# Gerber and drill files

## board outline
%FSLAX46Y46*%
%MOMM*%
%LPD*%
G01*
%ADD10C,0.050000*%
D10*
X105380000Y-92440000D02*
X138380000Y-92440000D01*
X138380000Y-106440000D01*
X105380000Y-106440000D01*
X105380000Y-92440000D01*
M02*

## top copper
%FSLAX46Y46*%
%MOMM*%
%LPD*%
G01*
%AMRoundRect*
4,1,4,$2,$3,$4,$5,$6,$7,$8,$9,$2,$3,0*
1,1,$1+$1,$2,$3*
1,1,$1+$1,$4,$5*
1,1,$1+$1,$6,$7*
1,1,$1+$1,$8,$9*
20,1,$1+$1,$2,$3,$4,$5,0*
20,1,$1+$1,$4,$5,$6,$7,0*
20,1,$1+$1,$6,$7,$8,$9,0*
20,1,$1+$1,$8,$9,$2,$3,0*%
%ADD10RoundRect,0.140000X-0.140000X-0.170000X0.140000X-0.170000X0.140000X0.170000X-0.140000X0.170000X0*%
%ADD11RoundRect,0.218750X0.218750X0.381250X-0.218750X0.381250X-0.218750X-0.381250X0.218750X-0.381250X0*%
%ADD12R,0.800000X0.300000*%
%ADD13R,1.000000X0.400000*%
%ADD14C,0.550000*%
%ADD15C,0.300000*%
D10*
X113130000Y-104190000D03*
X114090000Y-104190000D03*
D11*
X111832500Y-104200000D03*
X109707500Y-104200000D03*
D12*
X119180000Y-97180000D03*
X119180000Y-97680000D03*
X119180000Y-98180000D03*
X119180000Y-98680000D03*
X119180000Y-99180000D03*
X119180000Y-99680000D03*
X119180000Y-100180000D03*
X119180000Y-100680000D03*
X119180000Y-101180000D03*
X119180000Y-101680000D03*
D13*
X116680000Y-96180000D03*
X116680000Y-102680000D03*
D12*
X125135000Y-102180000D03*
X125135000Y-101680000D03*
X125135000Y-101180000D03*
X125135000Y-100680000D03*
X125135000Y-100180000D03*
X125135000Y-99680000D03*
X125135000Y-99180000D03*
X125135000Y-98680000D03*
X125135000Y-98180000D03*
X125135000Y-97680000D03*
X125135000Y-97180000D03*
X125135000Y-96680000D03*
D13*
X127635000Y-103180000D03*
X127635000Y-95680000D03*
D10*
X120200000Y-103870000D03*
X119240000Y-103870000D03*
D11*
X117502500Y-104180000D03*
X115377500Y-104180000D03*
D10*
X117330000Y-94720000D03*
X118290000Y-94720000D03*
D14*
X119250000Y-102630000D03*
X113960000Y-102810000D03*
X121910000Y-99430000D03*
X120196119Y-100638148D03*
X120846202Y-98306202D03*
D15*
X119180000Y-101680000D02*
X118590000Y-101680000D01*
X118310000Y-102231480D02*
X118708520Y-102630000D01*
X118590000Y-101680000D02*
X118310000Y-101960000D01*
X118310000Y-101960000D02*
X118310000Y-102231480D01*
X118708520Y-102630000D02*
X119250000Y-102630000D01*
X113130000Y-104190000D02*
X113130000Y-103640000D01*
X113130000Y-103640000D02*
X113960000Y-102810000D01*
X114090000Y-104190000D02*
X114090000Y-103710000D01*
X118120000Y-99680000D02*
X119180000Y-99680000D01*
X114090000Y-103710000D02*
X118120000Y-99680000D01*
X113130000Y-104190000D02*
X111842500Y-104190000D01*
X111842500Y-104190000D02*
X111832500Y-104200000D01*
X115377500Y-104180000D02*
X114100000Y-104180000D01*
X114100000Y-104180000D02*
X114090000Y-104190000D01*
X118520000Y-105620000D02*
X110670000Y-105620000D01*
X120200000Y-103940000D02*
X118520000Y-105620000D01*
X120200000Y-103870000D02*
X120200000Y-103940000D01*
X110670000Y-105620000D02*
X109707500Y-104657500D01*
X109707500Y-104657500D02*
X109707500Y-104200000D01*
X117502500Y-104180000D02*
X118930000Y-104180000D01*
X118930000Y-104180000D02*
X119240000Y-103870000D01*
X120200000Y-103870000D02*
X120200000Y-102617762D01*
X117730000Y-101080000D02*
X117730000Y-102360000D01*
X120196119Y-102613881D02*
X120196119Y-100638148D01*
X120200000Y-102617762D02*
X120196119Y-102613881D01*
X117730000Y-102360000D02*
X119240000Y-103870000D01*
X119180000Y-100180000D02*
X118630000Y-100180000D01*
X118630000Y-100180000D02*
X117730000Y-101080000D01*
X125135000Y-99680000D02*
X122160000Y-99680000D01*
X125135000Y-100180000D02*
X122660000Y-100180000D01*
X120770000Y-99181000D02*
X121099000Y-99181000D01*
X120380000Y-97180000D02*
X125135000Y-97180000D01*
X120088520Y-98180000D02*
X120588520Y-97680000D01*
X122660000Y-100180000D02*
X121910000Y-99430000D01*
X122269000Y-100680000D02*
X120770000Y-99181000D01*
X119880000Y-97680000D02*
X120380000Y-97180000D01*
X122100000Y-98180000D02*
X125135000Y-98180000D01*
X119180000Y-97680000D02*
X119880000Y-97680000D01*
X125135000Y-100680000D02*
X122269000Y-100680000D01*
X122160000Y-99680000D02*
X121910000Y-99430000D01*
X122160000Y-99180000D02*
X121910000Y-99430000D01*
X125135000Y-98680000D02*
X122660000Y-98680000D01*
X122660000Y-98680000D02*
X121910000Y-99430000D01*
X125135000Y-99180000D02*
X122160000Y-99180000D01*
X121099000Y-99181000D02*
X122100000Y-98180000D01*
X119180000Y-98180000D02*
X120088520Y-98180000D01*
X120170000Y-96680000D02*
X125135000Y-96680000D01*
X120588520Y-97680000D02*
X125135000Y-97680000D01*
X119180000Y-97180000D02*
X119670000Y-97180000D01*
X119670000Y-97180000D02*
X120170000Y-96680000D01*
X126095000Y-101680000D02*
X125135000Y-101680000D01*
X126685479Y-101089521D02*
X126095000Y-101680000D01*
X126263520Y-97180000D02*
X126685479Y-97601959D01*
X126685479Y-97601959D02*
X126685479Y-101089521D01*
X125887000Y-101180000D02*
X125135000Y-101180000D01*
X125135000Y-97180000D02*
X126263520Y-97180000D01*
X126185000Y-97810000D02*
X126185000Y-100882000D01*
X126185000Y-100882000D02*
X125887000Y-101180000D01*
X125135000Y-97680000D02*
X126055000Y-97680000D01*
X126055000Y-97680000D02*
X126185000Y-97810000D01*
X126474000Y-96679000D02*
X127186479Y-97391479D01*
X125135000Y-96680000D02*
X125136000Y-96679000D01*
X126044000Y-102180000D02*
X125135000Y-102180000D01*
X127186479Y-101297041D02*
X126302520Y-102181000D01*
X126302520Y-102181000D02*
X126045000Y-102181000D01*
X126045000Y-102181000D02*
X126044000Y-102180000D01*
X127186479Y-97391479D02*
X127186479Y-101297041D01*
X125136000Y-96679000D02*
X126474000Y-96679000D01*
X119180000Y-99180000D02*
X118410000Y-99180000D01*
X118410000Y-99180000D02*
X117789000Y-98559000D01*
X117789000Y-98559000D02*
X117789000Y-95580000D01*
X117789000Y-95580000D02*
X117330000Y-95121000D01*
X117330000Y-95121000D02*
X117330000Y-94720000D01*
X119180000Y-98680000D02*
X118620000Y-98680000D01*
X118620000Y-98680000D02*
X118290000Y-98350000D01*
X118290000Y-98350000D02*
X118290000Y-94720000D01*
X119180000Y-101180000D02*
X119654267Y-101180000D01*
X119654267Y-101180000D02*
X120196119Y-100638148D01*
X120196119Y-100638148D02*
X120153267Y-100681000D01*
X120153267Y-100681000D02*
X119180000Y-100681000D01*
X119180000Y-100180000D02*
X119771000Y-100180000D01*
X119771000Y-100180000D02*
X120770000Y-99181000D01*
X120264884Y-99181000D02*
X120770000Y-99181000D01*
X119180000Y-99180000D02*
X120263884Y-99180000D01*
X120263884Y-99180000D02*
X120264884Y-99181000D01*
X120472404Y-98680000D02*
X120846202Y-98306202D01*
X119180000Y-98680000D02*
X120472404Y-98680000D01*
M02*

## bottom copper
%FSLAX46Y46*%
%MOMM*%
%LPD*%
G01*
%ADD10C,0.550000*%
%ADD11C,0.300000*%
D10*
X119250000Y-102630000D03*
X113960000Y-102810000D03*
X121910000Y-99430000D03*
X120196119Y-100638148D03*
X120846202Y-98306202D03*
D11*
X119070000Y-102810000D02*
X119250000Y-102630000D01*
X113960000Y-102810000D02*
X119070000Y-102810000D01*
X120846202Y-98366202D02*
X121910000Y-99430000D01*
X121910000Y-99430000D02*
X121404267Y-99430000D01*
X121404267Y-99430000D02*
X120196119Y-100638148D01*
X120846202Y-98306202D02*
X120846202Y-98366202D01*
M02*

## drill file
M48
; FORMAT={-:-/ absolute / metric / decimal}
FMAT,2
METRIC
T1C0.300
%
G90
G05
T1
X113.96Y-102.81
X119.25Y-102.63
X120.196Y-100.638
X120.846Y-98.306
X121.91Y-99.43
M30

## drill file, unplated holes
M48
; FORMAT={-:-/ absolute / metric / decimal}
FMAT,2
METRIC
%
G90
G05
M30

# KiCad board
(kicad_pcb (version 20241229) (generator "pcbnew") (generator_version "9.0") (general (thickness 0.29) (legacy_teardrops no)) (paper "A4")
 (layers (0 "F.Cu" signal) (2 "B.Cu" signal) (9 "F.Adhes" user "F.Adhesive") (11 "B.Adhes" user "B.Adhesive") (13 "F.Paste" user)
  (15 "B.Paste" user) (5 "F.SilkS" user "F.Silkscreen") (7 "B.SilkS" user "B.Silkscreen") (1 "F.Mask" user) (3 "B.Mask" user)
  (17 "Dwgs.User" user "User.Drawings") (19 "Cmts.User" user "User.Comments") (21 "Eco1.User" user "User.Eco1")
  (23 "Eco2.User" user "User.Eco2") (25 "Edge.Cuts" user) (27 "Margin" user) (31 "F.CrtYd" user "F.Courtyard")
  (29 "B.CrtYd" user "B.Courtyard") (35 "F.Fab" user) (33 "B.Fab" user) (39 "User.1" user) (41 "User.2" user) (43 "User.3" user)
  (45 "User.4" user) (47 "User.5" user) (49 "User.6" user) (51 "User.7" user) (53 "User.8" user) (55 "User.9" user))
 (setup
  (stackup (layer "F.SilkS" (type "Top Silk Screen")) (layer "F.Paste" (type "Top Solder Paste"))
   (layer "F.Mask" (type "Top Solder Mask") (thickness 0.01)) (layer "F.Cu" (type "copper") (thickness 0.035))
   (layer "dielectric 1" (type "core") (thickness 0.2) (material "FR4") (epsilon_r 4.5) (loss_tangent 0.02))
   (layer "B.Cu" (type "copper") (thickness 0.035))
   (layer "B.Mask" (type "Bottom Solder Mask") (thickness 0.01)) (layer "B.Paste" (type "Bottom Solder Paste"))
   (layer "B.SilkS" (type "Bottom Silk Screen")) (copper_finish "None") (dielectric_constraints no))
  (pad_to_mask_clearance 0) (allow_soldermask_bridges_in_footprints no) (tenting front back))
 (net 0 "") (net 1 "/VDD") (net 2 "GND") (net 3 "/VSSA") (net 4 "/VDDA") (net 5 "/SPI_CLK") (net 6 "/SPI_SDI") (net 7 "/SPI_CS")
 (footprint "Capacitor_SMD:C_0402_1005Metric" (layer "F.Cu") (at 119.72 103.87)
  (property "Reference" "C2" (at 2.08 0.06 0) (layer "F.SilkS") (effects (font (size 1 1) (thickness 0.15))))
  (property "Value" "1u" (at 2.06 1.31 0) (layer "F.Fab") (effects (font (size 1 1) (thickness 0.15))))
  (pad "1" smd roundrect (at -0.48 0) (size 0.56 0.62) (layers "F.Cu" "F.Mask" "F.Paste") (roundrect_rratio 0.25) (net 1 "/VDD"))
  (pad "2" smd roundrect (at 0.48 0) (size 0.56 0.62) (layers "F.Cu" "F.Mask" "F.Paste") (roundrect_rratio 0.25) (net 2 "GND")))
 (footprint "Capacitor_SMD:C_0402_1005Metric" (layer "F.Cu") (at 113.61 104.19)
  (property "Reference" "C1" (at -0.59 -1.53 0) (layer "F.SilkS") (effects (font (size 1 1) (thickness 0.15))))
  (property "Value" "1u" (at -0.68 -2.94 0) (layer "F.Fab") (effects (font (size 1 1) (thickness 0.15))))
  (pad "1" smd roundrect (at -0.48 0) (size 0.56 0.62) (layers "F.Cu" "F.Mask" "F.Paste") (roundrect_rratio 0.25) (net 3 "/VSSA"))
  (pad "2" smd roundrect (at 0.48 0) (size 0.56 0.62) (layers "F.Cu" "F.Mask" "F.Paste") (roundrect_rratio 0.25) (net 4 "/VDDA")))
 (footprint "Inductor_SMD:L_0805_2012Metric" (layer "F.Cu") (at 116.44 104.18 180)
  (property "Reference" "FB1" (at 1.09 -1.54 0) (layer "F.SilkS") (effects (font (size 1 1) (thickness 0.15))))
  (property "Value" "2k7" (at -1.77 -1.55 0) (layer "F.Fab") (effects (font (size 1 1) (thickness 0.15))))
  (pad "1" smd roundrect (at -1.0625 0 180) (size 0.875 1.2) (layers "F.Cu" "F.Mask" "F.Paste") (roundrect_rratio 0.25) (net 1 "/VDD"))
  (pad "2" smd roundrect (at 1.0625 0 180) (size 0.875 1.2) (layers "F.Cu" "F.Mask" "F.Paste") (roundrect_rratio 0.25) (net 4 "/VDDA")))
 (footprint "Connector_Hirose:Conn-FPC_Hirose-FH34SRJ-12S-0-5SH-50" (layer "F.Cu") (at 126.16 99.43 90)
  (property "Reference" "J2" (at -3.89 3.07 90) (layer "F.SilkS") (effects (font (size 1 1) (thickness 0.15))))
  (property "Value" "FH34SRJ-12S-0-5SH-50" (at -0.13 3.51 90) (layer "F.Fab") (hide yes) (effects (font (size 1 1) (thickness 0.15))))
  (pad "1" smd rect (at -2.75 -1.025 90) (size 0.3 0.8) (layers "F.Cu" "F.Mask" "F.Paste") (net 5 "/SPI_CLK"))
  (pad "2" smd rect (at -2.25 -1.025 90) (size 0.3 0.8) (layers "F.Cu" "F.Mask" "F.Paste") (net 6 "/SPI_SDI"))
  (pad "3" smd rect (at -1.75 -1.025 90) (size 0.3 0.8) (layers "F.Cu" "F.Mask" "F.Paste") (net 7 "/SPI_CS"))
  (pad "4" smd rect (at -1.25 -1.025 90) (size 0.3 0.8) (layers "F.Cu" "F.Mask" "F.Paste") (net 1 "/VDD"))
  (pad "5" smd rect (at -0.75 -1.025 90) (size 0.3 0.8) (layers "F.Cu" "F.Mask" "F.Paste") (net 2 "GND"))
  (pad "6" smd rect (at -0.25 -1.025 90) (size 0.3 0.8) (layers "F.Cu" "F.Mask" "F.Paste") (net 2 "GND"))
  (pad "7" smd rect (at 0.25 -1.025 90) (size 0.3 0.8) (layers "F.Cu" "F.Mask" "F.Paste") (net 2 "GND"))
  (pad "8" smd rect (at 0.75 -1.025 90) (size 0.3 0.8) (layers "F.Cu" "F.Mask" "F.Paste") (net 2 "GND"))
  (pad "9" smd rect (at 1.25 -1.025 90) (size 0.3 0.8) (layers "F.Cu" "F.Mask" "F.Paste") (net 1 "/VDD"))
  (pad "10" smd rect (at 1.75 -1.025 90) (size 0.3 0.8) (layers "F.Cu" "F.Mask" "F.Paste") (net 7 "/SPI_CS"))
  (pad "11" smd rect (at 2.25 -1.025 90) (size 0.3 0.8) (layers "F.Cu" "F.Mask" "F.Paste") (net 6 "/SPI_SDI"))
  (pad "12" smd rect (at 2.75 -1.025 90) (size 0.3 0.8) (layers "F.Cu" "F.Mask" "F.Paste") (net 5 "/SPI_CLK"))
  (pad "MP" smd rect (at -3.75 1.475 90) (size 0.4 1) (layers "F.Cu" "F.Mask" "F.Paste"))
  (pad "MP" smd rect (at 3.75 1.475 90) (size 0.4 1) (layers "F.Cu" "F.Mask" "F.Paste")))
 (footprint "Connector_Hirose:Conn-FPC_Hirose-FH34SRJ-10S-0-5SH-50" (layer "F.Cu") (at 118.155 99.43 -90)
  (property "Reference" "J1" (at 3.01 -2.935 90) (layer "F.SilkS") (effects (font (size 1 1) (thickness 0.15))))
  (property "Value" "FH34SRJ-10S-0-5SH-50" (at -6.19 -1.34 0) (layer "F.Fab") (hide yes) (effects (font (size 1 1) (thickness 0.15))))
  (pad "1" smd rect (at -2.25 -1.025 270) (size 0.3 0.8) (layers "F.Cu" "F.Mask" "F.Paste") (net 5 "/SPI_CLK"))
  (pad "2" smd rect (at -1.75 -1.025 270) (size 0.3 0.8) (layers "F.Cu" "F.Mask" "F.Paste") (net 6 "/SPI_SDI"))
  (pad "3" smd rect (at -1.25 -1.025 270) (size 0.3 0.8) (layers "F.Cu" "F.Mask" "F.Paste") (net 7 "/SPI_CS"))
  (pad "4" smd rect (at -0.75 -1.025 270) (size 0.3 0.8) (layers "F.Cu" "F.Mask" "F.Paste") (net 2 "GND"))
  (pad "5" smd rect (at -0.25 -1.025 270) (size 0.3 0.8) (layers "F.Cu" "F.Mask" "F.Paste") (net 1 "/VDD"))
  (pad "6" smd rect (at 0.25 -1.025 270) (size 0.3 0.8) (layers "F.Cu" "F.Mask" "F.Paste") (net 4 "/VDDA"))
  (pad "7" smd rect (at 0.75 -1.025 270) (size 0.3 0.8) (layers "F.Cu" "F.Mask" "F.Paste") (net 1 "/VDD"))
  (pad "8" smd rect (at 1.25 -1.025 270) (size 0.3 0.8) (layers "F.Cu" "F.Mask" "F.Paste") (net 2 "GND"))
  (pad "9" smd rect (at 1.75 -1.025 270) (size 0.3 0.8) (layers "F.Cu" "F.Mask" "F.Paste") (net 2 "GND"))
  (pad "10" smd rect (at 2.25 -1.025 270) (size 0.3 0.8) (layers "F.Cu" "F.Mask" "F.Paste") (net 3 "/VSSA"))
  (pad "MP" smd rect (at -3.25 1.475 270) (size 0.4 1) (layers "F.Cu" "F.Mask" "F.Paste"))
  (pad "MP" smd rect (at 3.25 1.475 270) (size 0.4 1) (layers "F.Cu" "F.Mask" "F.Paste")))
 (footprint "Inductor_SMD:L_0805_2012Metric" (layer "F.Cu") (at 110.77 104.2 180)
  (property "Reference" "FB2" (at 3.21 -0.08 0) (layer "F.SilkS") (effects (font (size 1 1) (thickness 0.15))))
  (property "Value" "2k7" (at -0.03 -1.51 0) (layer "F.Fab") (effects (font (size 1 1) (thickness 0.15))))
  (pad "1" smd roundrect (at -1.0625 0 180) (size 0.875 1.2) (layers "F.Cu" "F.Mask" "F.Paste") (roundrect_rratio 0.25) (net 3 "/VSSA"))
  (pad "2" smd roundrect (at 1.0625 0 180) (size 0.875 1.2) (layers "F.Cu" "F.Mask" "F.Paste") (roundrect_rratio 0.25) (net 2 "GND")))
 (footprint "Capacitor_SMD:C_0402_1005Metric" (layer "F.Cu") (at 117.81 94.72)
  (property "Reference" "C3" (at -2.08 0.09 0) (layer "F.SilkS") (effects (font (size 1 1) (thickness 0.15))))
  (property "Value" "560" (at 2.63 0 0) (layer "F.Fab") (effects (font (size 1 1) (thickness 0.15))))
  (pad "1" smd roundrect (at -0.48 0) (size 0.56 0.62) (layers "F.Cu" "F.Mask" "F.Paste") (roundrect_rratio 0.25) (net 1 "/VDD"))
  (pad "2" smd roundrect (at 0.48 0) (size 0.56 0.62) (layers "F.Cu" "F.Mask" "F.Paste") (roundrect_rratio 0.25) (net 2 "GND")))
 (gr_rect (start 105.38 92.44) (end 138.38 106.44) (stroke (width 0.05) (type solid)) (fill no) (layer "Edge.Cuts"))
 (segment (start 115.3775 104.18) (end 114.1 104.18) (width 0.3) (layer "F.Cu") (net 4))
 (segment (start 114.09 104.19) (end 114.09 103.71) (width 0.3) (layer "F.Cu") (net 4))
 (segment (start 118.12 99.68) (end 119.18 99.68) (width 0.3) (layer "F.Cu") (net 4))
 (segment (start 114.1 104.18) (end 114.09 104.19) (width 0.3) (layer "F.Cu") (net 4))
 (segment (start 114.09 103.71) (end 118.12 99.68) (width 0.3) (layer "F.Cu") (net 4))
 (segment (start 118.31 102.23148) (end 118.70852 102.63) (width 0.3) (layer "F.Cu") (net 3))
 (segment (start 111.8425 104.19) (end 111.8325 104.2) (width 0.3) (layer "F.Cu") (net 3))
 (segment (start 118.70852 102.63) (end 119.25 102.63) (width 0.3) (layer "F.Cu") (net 3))
 (segment (start 119.18 101.68) (end 118.59 101.68) (width 0.3) (layer "F.Cu") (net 3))
 (segment (start 118.31 101.96) (end 118.31 102.23148) (width 0.3) (layer "F.Cu") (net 3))
 (segment (start 113.13 103.64) (end 113.96 102.81) (width 0.3) (layer "F.Cu") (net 3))
 (segment (start 118.59 101.68) (end 118.31 101.96) (width 0.3) (layer "F.Cu") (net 3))
 (segment (start 113.13 104.19) (end 113.13 103.64) (width 0.3) (layer "F.Cu") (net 3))
 (segment (start 113.13 104.19) (end 111.8425 104.19) (width 0.3) (layer "F.Cu") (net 3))
 (via (at 113.96 102.81) (size 0.55) (drill 0.3) (layers "F.Cu" "B.Cu") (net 3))
 (via (at 119.25 102.63) (size 0.55) (drill 0.3) (layers "F.Cu" "B.Cu") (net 3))
 (segment (start 113.96 102.81) (end 119.07 102.81) (width 0.3) (layer "B.Cu") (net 3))
 (segment (start 119.07 102.81) (end 119.25 102.63) (width 0.3) (layer "B.Cu") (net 3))
 (segment (start 120.472404 98.68) (end 120.846202 98.306202) (width 0.3) (layer "F.Cu") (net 2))
 (segment (start 120.2 103.87) (end 120.2 102.617762) (width 0.3) (layer "F.Cu") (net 2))
 (segment (start 120.153267 100.681) (end 119.18 100.681) (width 0.3) (layer "F.Cu") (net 2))
 (segment (start 120.2 103.94) (end 118.52 105.62) (width 0.3) (layer "F.Cu") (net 2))
 (segment (start 120.2 103.87) (end 120.2 103.94) (width 0.3) (layer "F.Cu") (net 2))
 (segment (start 125.135 98.68) (end 122.66 98.68) (width 0.3) (layer "F.Cu") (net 2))
 (segment (start 122.66 100.18) (end 121.91 99.43) (width 0.3) (layer "F.Cu") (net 2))
 (segment (start 119.18 98.68) (end 118.62 98.68) (width 0.3) (layer "F.Cu") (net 2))
 (segment (start 122.66 98.68) (end 121.91 99.43) (width 0.3) (layer "F.Cu") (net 2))
 (segment (start 125.135 100.18) (end 122.66 100.18) (width 0.3) (layer "F.Cu") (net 2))
 (segment (start 118.29 98.35) (end 118.29 94.72) (width 0.3) (layer "F.Cu") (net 2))
 (segment (start 119.18 98.68) (end 120.472404 98.68) (width 0.3) (layer "F.Cu") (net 2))
 (segment (start 125.135 99.18) (end 122.16 99.18) (width 0.3) (layer "F.Cu") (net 2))
 (segment (start 118.62 98.68) (end 118.29 98.35) (width 0.3) (layer "F.Cu") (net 2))
 (segment (start 120.2 102.617762) (end 120.196119 102.613881) (width 0.3) (layer "F.Cu") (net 2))
 (segment (start 122.16 99.18) (end 121.91 99.43) (width 0.3) (layer "F.Cu") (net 2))
 (segment (start 125.135 99.68) (end 122.16 99.68) (width 0.3) (layer "F.Cu") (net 2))
 (segment (start 119.654267 101.18) (end 120.196119 100.638148) (width 0.3) (layer "F.Cu") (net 2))
 (segment (start 122.16 99.68) (end 121.91 99.43) (width 0.3) (layer "F.Cu") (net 2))
 (segment (start 120.196119 102.613881) (end 120.196119 100.638148) (width 0.3) (layer "F.Cu") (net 2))
 (segment (start 110.67 105.62) (end 109.7075 104.6575) (width 0.3) (layer "F.Cu") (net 2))
 (segment (start 118.52 105.62) (end 110.67 105.62) (width 0.3) (layer "F.Cu") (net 2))
 (segment (start 109.7075 104.6575) (end 109.7075 104.2) (width 0.3) (layer "F.Cu") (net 2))
 (segment (start 119.18 101.18) (end 119.654267 101.18) (width 0.3) (layer "F.Cu") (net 2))
 (segment (start 120.196119 100.638148) (end 120.153267 100.681) (width 0.3) (layer "F.Cu") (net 2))
 (via (at 121.91 99.43) (size 0.55) (drill 0.3) (layers "F.Cu" "B.Cu") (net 2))
 (via (at 120.846202 98.306202) (size 0.55) (drill 0.3) (layers "F.Cu" "B.Cu") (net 2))
 (via (at 120.196119 100.638148) (size 0.55) (drill 0.3) (layers "F.Cu" "B.Cu") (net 2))
 (segment (start 120.846202 98.306202) (end 120.846202 98.366202) (width 0.3) (layer "B.Cu") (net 2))
 (segment (start 120.846202 98.366202) (end 121.91 99.43) (width 0.3) (layer "B.Cu") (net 2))
 (segment (start 121.404267 99.43) (end 120.196119 100.638148) (width 0.3) (layer "B.Cu") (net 2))
 (segment (start 121.91 99.43) (end 121.404267 99.43) (width 0.3) (layer "B.Cu") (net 2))
 (segment (start 125.135 100.68) (end 122.269 100.68) (width 0.3) (layer "F.Cu") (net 1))
 (segment (start 120.263884 99.18) (end 120.264884 99.181) (width 0.3) (layer "F.Cu") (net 1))
 (segment (start 119.18 99.18) (end 120.263884 99.18) (width 0.3) (layer "F.Cu") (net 1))
 (segment (start 119.18 100.18) (end 119.771 100.18) (width 0.3) (layer "F.Cu") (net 1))
 (segment (start 118.41 99.18) (end 117.789 98.559) (width 0.3) (layer "F.Cu") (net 1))
 (segment (start 122.1 98.18) (end 125.135 98.18) (width 0.3) (layer "F.Cu") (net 1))
 (segment (start 117.73 101.08) (end 117.73 102.36) (width 0.3) (layer "F.Cu") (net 1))
 (segment (start 118.93 104.18) (end 119.24 103.87) (width 0.3) (layer "F.Cu") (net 1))
 (segment (start 117.789 98.559) (end 117.789 95.58) (width 0.3) (layer "F.Cu") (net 1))
 (segment (start 117.73 102.36) (end 119.24 103.87) (width 0.3) (layer "F.Cu") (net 1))
 (segment (start 117.5025 104.18) (end 118.93 104.18) (width 0.3) (layer "F.Cu") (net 1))
 (segment (start 122.269 100.68) (end 120.77 99.181) (width 0.3) (layer "F.Cu") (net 1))
 (segment (start 119.771 100.18) (end 120.77 99.181) (width 0.3) (layer "F.Cu") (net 1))
 (segment (start 118.63 100.18) (end 117.73 101.08) (width 0.3) (layer "F.Cu") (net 1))
 (segment (start 117.789 95.58) (end 117.33 95.121) (width 0.3) (layer "F.Cu") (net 1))
 (segment (start 119.18 100.18) (end 118.63 100.18) (width 0.3) (layer "F.Cu") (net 1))
 (segment (start 117.33 95.121) (end 117.33 94.72) (width 0.3) (layer "F.Cu") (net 1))
 (segment (start 120.77 99.181) (end 121.099 99.181) (width 0.3) (layer "F.Cu") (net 1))
 (segment (start 119.18 99.18) (end 118.41 99.18) (width 0.3) (layer "F.Cu") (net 1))
 (segment (start 120.264884 99.181) (end 120.77 99.181) (width 0.3) (layer "F.Cu") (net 1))
 (segment (start 121.099 99.181) (end 122.1 98.18) (width 0.3) (layer "F.Cu") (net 1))
 (segment (start 119.18 98.18) (end 120.08852 98.18) (width 0.3) (layer "F.Cu") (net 7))
 (segment (start 126.055 97.68) (end 126.185 97.81) (width 0.3) (layer "F.Cu") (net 7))
 (segment (start 125.887 101.18) (end 125.135 101.18) (width 0.3) (layer "F.Cu") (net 7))
 (segment (start 126.185 97.81) (end 126.185 100.882) (width 0.3) (layer "F.Cu") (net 7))
 (segment (start 120.58852 97.68) (end 125.135 97.68) (width 0.3) (layer "F.Cu") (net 7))
 (segment (start 126.185 100.882) (end 125.887 101.18) (width 0.3) (layer "F.Cu") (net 7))
 (segment (start 125.135 97.68) (end 126.055 97.68) (width 0.3) (layer "F.Cu") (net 7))
 (segment (start 120.08852 98.18) (end 120.58852 97.68) (width 0.3) (layer "F.Cu") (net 7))
 (segment (start 120.38 97.18) (end 125.135 97.18) (width 0.3) (layer "F.Cu") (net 6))
 (segment (start 126.685479 97.601959) (end 126.685479 101.089521) (width 0.3) (layer "F.Cu") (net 6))
 (segment (start 125.135 97.18) (end 126.26352 97.18) (width 0.3) (layer "F.Cu") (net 6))
 (segment (start 119.18 97.68) (end 119.88 97.68) (width 0.3) (layer "F.Cu") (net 6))
 (segment (start 126.685479 101.089521) (end 126.095 101.68) (width 0.3) (layer "F.Cu") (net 6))
 (segment (start 126.095 101.68) (end 125.135 101.68) (width 0.3) (layer "F.Cu") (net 6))
 (segment (start 126.26352 97.18) (end 126.685479 97.601959) (width 0.3) (layer "F.Cu") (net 6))
 (segment (start 119.88 97.68) (end 120.38 97.18) (width 0.3) (layer "F.Cu") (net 6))
 (segment (start 127.186479 97.391479) (end 127.186479 101.297041) (width 0.3) (layer "F.Cu") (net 5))
 (segment (start 126.045 102.181) (end 126.044 102.18) (width 0.3) (layer "F.Cu") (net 5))
 (segment (start 119.67 97.18) (end 120.17 96.68) (width 0.3) (layer "F.Cu") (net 5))
 (segment (start 119.18 97.18) (end 119.67 97.18) (width 0.3) (layer "F.Cu") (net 5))
 (segment (start 125.135 96.68) (end 125.136 96.679) (width 0.3) (layer "F.Cu") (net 5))
 (segment (start 126.30252 102.181) (end 126.045 102.181) (width 0.3) (layer "F.Cu") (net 5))
 (segment (start 126.474 96.679) (end 127.186479 97.391479) (width 0.3) (layer "F.Cu") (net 5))
 (segment (start 126.044 102.18) (end 125.135 102.18) (width 0.3) (layer "F.Cu") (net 5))
 (segment (start 120.17 96.68) (end 125.135 96.68) (width 0.3) (layer "F.Cu") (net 5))
 (segment (start 127.186479 101.297041) (end 126.30252 102.181) (width 0.3) (layer "F.Cu") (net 5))
 (segment (start 125.136 96.679) (end 126.474 96.679) (width 0.3) (layer "F.Cu") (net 5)))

